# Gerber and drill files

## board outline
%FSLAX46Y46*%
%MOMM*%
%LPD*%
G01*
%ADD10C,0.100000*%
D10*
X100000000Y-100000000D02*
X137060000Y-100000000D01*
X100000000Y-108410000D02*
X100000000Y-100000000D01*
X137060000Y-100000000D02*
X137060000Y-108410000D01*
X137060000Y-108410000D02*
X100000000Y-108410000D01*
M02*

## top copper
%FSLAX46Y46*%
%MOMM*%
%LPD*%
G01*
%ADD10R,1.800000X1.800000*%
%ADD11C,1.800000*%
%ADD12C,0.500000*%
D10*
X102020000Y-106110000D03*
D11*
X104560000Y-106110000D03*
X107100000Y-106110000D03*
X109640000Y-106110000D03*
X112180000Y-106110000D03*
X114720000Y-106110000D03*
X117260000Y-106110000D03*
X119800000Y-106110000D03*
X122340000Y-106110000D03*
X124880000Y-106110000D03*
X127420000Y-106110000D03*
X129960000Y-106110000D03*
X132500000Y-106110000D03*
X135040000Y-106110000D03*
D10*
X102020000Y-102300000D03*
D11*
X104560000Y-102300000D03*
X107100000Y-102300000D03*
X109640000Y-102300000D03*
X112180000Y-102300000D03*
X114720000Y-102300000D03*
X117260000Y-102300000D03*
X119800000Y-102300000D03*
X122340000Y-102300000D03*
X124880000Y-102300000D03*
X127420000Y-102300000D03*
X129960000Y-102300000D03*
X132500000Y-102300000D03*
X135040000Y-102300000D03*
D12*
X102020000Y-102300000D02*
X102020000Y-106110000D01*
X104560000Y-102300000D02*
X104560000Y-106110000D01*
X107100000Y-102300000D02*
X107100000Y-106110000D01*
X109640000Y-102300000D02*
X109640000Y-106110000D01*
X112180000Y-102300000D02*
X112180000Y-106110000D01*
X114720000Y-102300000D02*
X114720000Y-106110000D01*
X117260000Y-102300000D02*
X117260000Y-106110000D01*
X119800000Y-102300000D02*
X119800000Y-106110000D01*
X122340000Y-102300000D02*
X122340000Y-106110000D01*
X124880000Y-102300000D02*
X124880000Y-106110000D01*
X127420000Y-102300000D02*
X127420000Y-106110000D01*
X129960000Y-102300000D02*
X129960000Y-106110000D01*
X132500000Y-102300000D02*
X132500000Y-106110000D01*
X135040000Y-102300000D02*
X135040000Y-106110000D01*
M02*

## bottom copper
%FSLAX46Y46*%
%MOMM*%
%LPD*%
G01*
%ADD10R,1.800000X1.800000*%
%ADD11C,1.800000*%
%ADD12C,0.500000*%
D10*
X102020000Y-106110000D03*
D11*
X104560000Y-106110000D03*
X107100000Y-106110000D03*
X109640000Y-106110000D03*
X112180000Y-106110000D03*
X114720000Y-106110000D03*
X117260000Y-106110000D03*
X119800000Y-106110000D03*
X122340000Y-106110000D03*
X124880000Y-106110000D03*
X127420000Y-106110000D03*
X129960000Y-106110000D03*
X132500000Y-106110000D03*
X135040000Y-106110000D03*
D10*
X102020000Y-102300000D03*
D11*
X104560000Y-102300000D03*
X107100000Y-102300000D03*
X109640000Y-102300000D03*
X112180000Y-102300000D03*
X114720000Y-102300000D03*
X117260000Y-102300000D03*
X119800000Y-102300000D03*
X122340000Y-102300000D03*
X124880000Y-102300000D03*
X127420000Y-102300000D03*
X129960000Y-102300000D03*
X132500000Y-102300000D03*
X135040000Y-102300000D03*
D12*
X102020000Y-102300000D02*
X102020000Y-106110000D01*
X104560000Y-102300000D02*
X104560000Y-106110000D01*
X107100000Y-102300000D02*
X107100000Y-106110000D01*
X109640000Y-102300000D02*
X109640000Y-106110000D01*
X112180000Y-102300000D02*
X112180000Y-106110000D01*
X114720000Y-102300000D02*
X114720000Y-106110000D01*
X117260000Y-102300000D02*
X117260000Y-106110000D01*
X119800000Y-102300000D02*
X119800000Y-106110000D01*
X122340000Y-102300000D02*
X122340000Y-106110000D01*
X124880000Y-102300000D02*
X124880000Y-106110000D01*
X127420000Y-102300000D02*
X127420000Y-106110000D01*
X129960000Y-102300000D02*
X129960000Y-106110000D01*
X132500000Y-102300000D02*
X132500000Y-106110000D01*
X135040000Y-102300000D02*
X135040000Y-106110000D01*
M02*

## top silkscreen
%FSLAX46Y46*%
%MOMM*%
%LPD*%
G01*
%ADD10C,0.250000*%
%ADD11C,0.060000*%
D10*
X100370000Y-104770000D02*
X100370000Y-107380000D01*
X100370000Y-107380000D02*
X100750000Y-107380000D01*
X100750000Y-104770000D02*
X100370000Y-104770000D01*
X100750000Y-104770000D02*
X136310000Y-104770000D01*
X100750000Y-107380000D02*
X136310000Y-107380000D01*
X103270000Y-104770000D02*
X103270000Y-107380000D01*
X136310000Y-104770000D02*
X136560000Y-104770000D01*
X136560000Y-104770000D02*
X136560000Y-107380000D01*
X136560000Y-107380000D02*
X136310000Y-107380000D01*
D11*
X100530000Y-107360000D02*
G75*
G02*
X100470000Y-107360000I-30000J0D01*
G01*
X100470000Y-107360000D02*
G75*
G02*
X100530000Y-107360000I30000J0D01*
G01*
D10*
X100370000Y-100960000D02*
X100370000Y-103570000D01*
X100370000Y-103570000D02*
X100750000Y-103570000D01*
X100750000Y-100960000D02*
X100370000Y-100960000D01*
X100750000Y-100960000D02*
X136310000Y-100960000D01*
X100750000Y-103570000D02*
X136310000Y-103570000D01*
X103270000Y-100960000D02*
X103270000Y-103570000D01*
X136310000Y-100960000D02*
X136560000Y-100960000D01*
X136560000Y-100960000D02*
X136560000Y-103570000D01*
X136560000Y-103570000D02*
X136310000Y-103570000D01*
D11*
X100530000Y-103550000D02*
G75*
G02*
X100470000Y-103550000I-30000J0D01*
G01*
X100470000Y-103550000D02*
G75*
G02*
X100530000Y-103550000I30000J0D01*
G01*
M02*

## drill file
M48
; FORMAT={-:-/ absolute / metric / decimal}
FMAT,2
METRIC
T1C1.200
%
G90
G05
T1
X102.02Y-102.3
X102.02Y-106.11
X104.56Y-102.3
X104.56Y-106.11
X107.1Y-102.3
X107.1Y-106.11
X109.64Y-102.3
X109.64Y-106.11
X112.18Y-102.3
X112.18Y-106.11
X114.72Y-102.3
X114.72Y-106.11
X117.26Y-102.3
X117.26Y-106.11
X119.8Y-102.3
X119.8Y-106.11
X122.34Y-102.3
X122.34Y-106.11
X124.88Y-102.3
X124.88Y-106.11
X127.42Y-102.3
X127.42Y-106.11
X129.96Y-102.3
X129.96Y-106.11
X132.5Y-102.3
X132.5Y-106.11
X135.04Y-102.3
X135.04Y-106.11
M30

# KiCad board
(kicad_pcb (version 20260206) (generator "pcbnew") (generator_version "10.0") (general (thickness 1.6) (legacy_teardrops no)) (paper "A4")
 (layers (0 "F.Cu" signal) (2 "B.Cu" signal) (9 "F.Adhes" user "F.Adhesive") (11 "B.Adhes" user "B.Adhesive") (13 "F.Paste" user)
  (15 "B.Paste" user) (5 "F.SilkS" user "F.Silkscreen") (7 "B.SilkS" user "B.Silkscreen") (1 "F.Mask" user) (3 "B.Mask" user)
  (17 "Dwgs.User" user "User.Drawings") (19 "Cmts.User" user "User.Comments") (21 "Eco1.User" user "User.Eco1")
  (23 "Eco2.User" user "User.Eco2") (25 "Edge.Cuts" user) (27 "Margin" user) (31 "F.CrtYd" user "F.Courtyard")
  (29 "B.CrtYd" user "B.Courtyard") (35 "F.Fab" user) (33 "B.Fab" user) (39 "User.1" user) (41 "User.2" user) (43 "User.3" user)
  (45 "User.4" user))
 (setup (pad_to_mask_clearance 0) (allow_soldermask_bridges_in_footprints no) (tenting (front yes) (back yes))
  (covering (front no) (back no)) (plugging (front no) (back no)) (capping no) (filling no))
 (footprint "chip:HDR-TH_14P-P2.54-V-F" (layer "F.Cu") (at 118.53 106.11)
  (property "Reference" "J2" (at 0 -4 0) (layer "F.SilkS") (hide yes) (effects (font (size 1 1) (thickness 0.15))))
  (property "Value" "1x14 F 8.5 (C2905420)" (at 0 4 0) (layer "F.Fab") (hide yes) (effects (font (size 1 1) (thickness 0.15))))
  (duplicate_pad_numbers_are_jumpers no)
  (fp_line (start -18.16 -1.34) (end -18.16 1.27) (stroke (width 0.25) (type solid)) (layer "F.SilkS"))
  (fp_line (start -18.16 1.27) (end -17.78 1.27) (stroke (width 0.25) (type solid)) (layer "F.SilkS"))
  (fp_line (start -17.78 -1.34) (end -18.16 -1.34) (stroke (width 0.25) (type solid)) (layer "F.SilkS"))
  (fp_line (start -17.78 -1.34) (end 17.78 -1.34) (stroke (width 0.25) (type solid)) (layer "F.SilkS"))
  (fp_line (start -17.78 1.27) (end 17.78 1.27) (stroke (width 0.25) (type solid)) (layer "F.SilkS"))
  (fp_line (start -15.26 -1.34) (end -15.26 1.27) (stroke (width 0.25) (type solid)) (layer "F.SilkS"))
  (fp_line (start 17.78 -1.34) (end 18.03 -1.34) (stroke (width 0.25) (type solid)) (layer "F.SilkS"))
  (fp_line (start 18.03 -1.34) (end 18.03 1.27) (stroke (width 0.25) (type solid)) (layer "F.SilkS"))
  (fp_line (start 18.03 1.27) (end 17.78 1.27) (stroke (width 0.25) (type solid)) (layer "F.SilkS"))
  (fp_circle (center -18.03 1.25) (end -18 1.25) (stroke (width 0.06) (type solid)) (fill no) (layer "F.SilkS"))
  (pad "1" thru_hole rect (at -16.51 0) (size 1.8 1.8) (drill 1.199998) (layers "*.Cu" "*.Mask") (remove_unused_layers no) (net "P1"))
  (pad "2" thru_hole circle (at -13.97 0) (size 1.8 1.8) (drill 1.199998) (layers "*.Cu" "*.Mask") (remove_unused_layers no) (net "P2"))
  (pad "3" thru_hole circle (at -11.43 0) (size 1.8 1.8) (drill 1.199998) (layers "*.Cu" "*.Mask") (remove_unused_layers no) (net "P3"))
  (pad "4" thru_hole circle (at -8.89 0) (size 1.8 1.8) (drill 1.199998) (layers "*.Cu" "*.Mask") (remove_unused_layers no) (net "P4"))
  (pad "5" thru_hole circle (at -6.35 0) (size 1.8 1.8) (drill 1.199998) (layers "*.Cu" "*.Mask") (remove_unused_layers no) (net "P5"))
  (pad "6" thru_hole circle (at -3.81 0) (size 1.8 1.8) (drill 1.199998) (layers "*.Cu" "*.Mask") (remove_unused_layers no) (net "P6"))
  (pad "7" thru_hole circle (at -1.27 0) (size 1.8 1.8) (drill 1.199998) (layers "*.Cu" "*.Mask") (remove_unused_layers no) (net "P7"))
  (pad "8" thru_hole circle (at 1.27 0) (size 1.8 1.8) (drill 1.199998) (layers "*.Cu" "*.Mask") (remove_unused_layers no) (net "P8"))
  (pad "9" thru_hole circle (at 3.81 0) (size 1.8 1.8) (drill 1.199998) (layers "*.Cu" "*.Mask") (remove_unused_layers no) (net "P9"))
  (pad "10" thru_hole circle (at 6.35 0) (size 1.8 1.8) (drill 1.199998) (layers "*.Cu" "*.Mask") (remove_unused_layers no) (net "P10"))
  (pad "11" thru_hole circle (at 8.89 0) (size 1.8 1.8) (drill 1.199998) (layers "*.Cu" "*.Mask") (remove_unused_layers no) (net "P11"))
  (pad "12" thru_hole circle (at 11.43 0) (size 1.8 1.8) (drill 1.199998) (layers "*.Cu" "*.Mask") (remove_unused_layers no) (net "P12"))
  (pad "13" thru_hole circle (at 13.97 0) (size 1.8 1.8) (drill 1.199998) (layers "*.Cu" "*.Mask") (remove_unused_layers no) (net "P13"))
  (pad "14" thru_hole circle (at 16.51 0) (size 1.8 1.8) (drill 1.199998) (layers "*.Cu" "*.Mask") (remove_unused_layers no) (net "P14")))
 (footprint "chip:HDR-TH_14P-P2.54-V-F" (layer "F.Cu") (at 118.53 102.3)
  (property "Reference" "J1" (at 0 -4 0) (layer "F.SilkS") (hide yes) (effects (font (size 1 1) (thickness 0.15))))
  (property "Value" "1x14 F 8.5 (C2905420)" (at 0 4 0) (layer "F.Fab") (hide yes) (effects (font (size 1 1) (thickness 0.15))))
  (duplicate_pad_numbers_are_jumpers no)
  (fp_line (start -18.16 -1.34) (end -18.16 1.27) (stroke (width 0.25) (type solid)) (layer "F.SilkS"))
  (fp_line (start -18.16 1.27) (end -17.78 1.27) (stroke (width 0.25) (type solid)) (layer "F.SilkS"))
  (fp_line (start -17.78 -1.34) (end -18.16 -1.34) (stroke (width 0.25) (type solid)) (layer "F.SilkS"))
  (fp_line (start -17.78 -1.34) (end 17.78 -1.34) (stroke (width 0.25) (type solid)) (layer "F.SilkS"))
  (fp_line (start -17.78 1.27) (end 17.78 1.27) (stroke (width 0.25) (type solid)) (layer "F.SilkS"))
  (fp_line (start -15.26 -1.34) (end -15.26 1.27) (stroke (width 0.25) (type solid)) (layer "F.SilkS"))
  (fp_line (start 17.78 -1.34) (end 18.03 -1.34) (stroke (width 0.25) (type solid)) (layer "F.SilkS"))
  (fp_line (start 18.03 -1.34) (end 18.03 1.27) (stroke (width 0.25) (type solid)) (layer "F.SilkS"))
  (fp_line (start 18.03 1.27) (end 17.78 1.27) (stroke (width 0.25) (type solid)) (layer "F.SilkS"))
  (fp_circle (center -18.03 1.25) (end -18 1.25) (stroke (width 0.06) (type solid)) (fill no) (layer "F.SilkS"))
  (pad "1" thru_hole rect (at -16.51 0) (size 1.8 1.8) (drill 1.199998) (layers "*.Cu" "*.Mask") (remove_unused_layers no) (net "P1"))
  (pad "2" thru_hole circle (at -13.97 0) (size 1.8 1.8) (drill 1.199998) (layers "*.Cu" "*.Mask") (remove_unused_layers no) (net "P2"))
  (pad "3" thru_hole circle (at -11.43 0) (size 1.8 1.8) (drill 1.199998) (layers "*.Cu" "*.Mask") (remove_unused_layers no) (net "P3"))
  (pad "4" thru_hole circle (at -8.89 0) (size 1.8 1.8) (drill 1.199998) (layers "*.Cu" "*.Mask") (remove_unused_layers no) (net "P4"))
  (pad "5" thru_hole circle (at -6.35 0) (size 1.8 1.8) (drill 1.199998) (layers "*.Cu" "*.Mask") (remove_unused_layers no) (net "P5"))
  (pad "6" thru_hole circle (at -3.81 0) (size 1.8 1.8) (drill 1.199998) (layers "*.Cu" "*.Mask") (remove_unused_layers no) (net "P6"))
  (pad "7" thru_hole circle (at -1.27 0) (size 1.8 1.8) (drill 1.199998) (layers "*.Cu" "*.Mask") (remove_unused_layers no) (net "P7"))
  (pad "8" thru_hole circle (at 1.27 0) (size 1.8 1.8) (drill 1.199998) (layers "*.Cu" "*.Mask") (remove_unused_layers no) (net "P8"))
  (pad "9" thru_hole circle (at 3.81 0) (size 1.8 1.8) (drill 1.199998) (layers "*.Cu" "*.Mask") (remove_unused_layers no) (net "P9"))
  (pad "10" thru_hole circle (at 6.35 0) (size 1.8 1.8) (drill 1.199998) (layers "*.Cu" "*.Mask") (remove_unused_layers no) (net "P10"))
  (pad "11" thru_hole circle (at 8.89 0) (size 1.8 1.8) (drill 1.199998) (layers "*.Cu" "*.Mask") (remove_unused_layers no) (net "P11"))
  (pad "12" thru_hole circle (at 11.43 0) (size 1.8 1.8) (drill 1.199998) (layers "*.Cu" "*.Mask") (remove_unused_layers no) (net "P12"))
  (pad "13" thru_hole circle (at 13.97 0) (size 1.8 1.8) (drill 1.199998) (layers "*.Cu" "*.Mask") (remove_unused_layers no) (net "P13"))
  (pad "14" thru_hole circle (at 16.51 0) (size 1.8 1.8) (drill 1.199998) (layers "*.Cu" "*.Mask") (remove_unused_layers no) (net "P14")))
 (gr_line (start 100 100) (end 137.06 100) (stroke (width 0.1) (type default)) (layer "Edge.Cuts"))
 (gr_line (start 100 108.41) (end 100 100) (stroke (width 0.1) (type default)) (layer "Edge.Cuts"))
 (gr_line (start 137.06 100) (end 137.06 108.41) (stroke (width 0.1) (type default)) (layer "Edge.Cuts"))
 (gr_line (start 137.06 108.41) (end 100 108.41) (stroke (width 0.1) (type default)) (layer "Edge.Cuts"))
 (segment (start 102.02 102.3) (end 102.02 106.11) (width 0.5) (layer "F.Cu") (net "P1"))
 (segment (start 102.02 102.3) (end 102.02 106.11) (width 0.5) (layer "B.Cu") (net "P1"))
 (segment (start 104.56 102.3) (end 104.56 106.11) (width 0.5) (layer "F.Cu") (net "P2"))
 (segment (start 104.56 102.3) (end 104.56 106.11) (width 0.5) (layer "B.Cu") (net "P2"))
 (segment (start 107.1 102.3) (end 107.1 106.11) (width 0.5) (layer "F.Cu") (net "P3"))
 (segment (start 107.1 102.3) (end 107.1 106.11) (width 0.5) (layer "B.Cu") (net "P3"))
 (segment (start 109.64 102.3) (end 109.64 106.11) (width 0.5) (layer "F.Cu") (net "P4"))
 (segment (start 109.64 102.3) (end 109.64 106.11) (width 0.5) (layer "B.Cu") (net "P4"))
 (segment (start 112.18 102.3) (end 112.18 106.11) (width 0.5) (layer "F.Cu") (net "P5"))
 (segment (start 112.18 102.3) (end 112.18 106.11) (width 0.5) (layer "B.Cu") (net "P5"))
 (segment (start 114.72 102.3) (end 114.72 106.11) (width 0.5) (layer "F.Cu") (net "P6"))
 (segment (start 114.72 102.3) (end 114.72 106.11) (width 0.5) (layer "B.Cu") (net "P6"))
 (segment (start 117.26 102.3) (end 117.26 106.11) (width 0.5) (layer "F.Cu") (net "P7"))
 (segment (start 117.26 102.3) (end 117.26 106.11) (width 0.5) (layer "B.Cu") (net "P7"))
 (segment (start 119.8 102.3) (end 119.8 106.11) (width 0.5) (layer "F.Cu") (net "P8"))
 (segment (start 119.8 102.3) (end 119.8 106.11) (width 0.5) (layer "B.Cu") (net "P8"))
 (segment (start 122.34 102.3) (end 122.34 106.11) (width 0.5) (layer "F.Cu") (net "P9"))
 (segment (start 122.34 102.3) (end 122.34 106.11) (width 0.5) (layer "B.Cu") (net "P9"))
 (segment (start 124.88 102.3) (end 124.88 106.11) (width 0.5) (layer "F.Cu") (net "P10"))
 (segment (start 124.88 102.3) (end 124.88 106.11) (width 0.5) (layer "B.Cu") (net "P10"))
 (segment (start 127.42 102.3) (end 127.42 106.11) (width 0.5) (layer "F.Cu") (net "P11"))
 (segment (start 127.42 102.3) (end 127.42 106.11) (width 0.5) (layer "B.Cu") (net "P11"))
 (segment (start 129.96 102.3) (end 129.96 106.11) (width 0.5) (layer "F.Cu") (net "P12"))
 (segment (start 129.96 102.3) (end 129.96 106.11) (width 0.5) (layer "B.Cu") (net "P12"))
 (segment (start 132.5 102.3) (end 132.5 106.11) (width 0.5) (layer "F.Cu") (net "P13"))
 (segment (start 132.5 102.3) (end 132.5 106.11) (width 0.5) (layer "B.Cu") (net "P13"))
 (segment (start 135.04 102.3) (end 135.04 106.11) (width 0.5) (layer "F.Cu") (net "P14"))
 (segment (start 135.04 102.3) (end 135.04 106.11) (width 0.5) (layer "B.Cu") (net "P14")))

